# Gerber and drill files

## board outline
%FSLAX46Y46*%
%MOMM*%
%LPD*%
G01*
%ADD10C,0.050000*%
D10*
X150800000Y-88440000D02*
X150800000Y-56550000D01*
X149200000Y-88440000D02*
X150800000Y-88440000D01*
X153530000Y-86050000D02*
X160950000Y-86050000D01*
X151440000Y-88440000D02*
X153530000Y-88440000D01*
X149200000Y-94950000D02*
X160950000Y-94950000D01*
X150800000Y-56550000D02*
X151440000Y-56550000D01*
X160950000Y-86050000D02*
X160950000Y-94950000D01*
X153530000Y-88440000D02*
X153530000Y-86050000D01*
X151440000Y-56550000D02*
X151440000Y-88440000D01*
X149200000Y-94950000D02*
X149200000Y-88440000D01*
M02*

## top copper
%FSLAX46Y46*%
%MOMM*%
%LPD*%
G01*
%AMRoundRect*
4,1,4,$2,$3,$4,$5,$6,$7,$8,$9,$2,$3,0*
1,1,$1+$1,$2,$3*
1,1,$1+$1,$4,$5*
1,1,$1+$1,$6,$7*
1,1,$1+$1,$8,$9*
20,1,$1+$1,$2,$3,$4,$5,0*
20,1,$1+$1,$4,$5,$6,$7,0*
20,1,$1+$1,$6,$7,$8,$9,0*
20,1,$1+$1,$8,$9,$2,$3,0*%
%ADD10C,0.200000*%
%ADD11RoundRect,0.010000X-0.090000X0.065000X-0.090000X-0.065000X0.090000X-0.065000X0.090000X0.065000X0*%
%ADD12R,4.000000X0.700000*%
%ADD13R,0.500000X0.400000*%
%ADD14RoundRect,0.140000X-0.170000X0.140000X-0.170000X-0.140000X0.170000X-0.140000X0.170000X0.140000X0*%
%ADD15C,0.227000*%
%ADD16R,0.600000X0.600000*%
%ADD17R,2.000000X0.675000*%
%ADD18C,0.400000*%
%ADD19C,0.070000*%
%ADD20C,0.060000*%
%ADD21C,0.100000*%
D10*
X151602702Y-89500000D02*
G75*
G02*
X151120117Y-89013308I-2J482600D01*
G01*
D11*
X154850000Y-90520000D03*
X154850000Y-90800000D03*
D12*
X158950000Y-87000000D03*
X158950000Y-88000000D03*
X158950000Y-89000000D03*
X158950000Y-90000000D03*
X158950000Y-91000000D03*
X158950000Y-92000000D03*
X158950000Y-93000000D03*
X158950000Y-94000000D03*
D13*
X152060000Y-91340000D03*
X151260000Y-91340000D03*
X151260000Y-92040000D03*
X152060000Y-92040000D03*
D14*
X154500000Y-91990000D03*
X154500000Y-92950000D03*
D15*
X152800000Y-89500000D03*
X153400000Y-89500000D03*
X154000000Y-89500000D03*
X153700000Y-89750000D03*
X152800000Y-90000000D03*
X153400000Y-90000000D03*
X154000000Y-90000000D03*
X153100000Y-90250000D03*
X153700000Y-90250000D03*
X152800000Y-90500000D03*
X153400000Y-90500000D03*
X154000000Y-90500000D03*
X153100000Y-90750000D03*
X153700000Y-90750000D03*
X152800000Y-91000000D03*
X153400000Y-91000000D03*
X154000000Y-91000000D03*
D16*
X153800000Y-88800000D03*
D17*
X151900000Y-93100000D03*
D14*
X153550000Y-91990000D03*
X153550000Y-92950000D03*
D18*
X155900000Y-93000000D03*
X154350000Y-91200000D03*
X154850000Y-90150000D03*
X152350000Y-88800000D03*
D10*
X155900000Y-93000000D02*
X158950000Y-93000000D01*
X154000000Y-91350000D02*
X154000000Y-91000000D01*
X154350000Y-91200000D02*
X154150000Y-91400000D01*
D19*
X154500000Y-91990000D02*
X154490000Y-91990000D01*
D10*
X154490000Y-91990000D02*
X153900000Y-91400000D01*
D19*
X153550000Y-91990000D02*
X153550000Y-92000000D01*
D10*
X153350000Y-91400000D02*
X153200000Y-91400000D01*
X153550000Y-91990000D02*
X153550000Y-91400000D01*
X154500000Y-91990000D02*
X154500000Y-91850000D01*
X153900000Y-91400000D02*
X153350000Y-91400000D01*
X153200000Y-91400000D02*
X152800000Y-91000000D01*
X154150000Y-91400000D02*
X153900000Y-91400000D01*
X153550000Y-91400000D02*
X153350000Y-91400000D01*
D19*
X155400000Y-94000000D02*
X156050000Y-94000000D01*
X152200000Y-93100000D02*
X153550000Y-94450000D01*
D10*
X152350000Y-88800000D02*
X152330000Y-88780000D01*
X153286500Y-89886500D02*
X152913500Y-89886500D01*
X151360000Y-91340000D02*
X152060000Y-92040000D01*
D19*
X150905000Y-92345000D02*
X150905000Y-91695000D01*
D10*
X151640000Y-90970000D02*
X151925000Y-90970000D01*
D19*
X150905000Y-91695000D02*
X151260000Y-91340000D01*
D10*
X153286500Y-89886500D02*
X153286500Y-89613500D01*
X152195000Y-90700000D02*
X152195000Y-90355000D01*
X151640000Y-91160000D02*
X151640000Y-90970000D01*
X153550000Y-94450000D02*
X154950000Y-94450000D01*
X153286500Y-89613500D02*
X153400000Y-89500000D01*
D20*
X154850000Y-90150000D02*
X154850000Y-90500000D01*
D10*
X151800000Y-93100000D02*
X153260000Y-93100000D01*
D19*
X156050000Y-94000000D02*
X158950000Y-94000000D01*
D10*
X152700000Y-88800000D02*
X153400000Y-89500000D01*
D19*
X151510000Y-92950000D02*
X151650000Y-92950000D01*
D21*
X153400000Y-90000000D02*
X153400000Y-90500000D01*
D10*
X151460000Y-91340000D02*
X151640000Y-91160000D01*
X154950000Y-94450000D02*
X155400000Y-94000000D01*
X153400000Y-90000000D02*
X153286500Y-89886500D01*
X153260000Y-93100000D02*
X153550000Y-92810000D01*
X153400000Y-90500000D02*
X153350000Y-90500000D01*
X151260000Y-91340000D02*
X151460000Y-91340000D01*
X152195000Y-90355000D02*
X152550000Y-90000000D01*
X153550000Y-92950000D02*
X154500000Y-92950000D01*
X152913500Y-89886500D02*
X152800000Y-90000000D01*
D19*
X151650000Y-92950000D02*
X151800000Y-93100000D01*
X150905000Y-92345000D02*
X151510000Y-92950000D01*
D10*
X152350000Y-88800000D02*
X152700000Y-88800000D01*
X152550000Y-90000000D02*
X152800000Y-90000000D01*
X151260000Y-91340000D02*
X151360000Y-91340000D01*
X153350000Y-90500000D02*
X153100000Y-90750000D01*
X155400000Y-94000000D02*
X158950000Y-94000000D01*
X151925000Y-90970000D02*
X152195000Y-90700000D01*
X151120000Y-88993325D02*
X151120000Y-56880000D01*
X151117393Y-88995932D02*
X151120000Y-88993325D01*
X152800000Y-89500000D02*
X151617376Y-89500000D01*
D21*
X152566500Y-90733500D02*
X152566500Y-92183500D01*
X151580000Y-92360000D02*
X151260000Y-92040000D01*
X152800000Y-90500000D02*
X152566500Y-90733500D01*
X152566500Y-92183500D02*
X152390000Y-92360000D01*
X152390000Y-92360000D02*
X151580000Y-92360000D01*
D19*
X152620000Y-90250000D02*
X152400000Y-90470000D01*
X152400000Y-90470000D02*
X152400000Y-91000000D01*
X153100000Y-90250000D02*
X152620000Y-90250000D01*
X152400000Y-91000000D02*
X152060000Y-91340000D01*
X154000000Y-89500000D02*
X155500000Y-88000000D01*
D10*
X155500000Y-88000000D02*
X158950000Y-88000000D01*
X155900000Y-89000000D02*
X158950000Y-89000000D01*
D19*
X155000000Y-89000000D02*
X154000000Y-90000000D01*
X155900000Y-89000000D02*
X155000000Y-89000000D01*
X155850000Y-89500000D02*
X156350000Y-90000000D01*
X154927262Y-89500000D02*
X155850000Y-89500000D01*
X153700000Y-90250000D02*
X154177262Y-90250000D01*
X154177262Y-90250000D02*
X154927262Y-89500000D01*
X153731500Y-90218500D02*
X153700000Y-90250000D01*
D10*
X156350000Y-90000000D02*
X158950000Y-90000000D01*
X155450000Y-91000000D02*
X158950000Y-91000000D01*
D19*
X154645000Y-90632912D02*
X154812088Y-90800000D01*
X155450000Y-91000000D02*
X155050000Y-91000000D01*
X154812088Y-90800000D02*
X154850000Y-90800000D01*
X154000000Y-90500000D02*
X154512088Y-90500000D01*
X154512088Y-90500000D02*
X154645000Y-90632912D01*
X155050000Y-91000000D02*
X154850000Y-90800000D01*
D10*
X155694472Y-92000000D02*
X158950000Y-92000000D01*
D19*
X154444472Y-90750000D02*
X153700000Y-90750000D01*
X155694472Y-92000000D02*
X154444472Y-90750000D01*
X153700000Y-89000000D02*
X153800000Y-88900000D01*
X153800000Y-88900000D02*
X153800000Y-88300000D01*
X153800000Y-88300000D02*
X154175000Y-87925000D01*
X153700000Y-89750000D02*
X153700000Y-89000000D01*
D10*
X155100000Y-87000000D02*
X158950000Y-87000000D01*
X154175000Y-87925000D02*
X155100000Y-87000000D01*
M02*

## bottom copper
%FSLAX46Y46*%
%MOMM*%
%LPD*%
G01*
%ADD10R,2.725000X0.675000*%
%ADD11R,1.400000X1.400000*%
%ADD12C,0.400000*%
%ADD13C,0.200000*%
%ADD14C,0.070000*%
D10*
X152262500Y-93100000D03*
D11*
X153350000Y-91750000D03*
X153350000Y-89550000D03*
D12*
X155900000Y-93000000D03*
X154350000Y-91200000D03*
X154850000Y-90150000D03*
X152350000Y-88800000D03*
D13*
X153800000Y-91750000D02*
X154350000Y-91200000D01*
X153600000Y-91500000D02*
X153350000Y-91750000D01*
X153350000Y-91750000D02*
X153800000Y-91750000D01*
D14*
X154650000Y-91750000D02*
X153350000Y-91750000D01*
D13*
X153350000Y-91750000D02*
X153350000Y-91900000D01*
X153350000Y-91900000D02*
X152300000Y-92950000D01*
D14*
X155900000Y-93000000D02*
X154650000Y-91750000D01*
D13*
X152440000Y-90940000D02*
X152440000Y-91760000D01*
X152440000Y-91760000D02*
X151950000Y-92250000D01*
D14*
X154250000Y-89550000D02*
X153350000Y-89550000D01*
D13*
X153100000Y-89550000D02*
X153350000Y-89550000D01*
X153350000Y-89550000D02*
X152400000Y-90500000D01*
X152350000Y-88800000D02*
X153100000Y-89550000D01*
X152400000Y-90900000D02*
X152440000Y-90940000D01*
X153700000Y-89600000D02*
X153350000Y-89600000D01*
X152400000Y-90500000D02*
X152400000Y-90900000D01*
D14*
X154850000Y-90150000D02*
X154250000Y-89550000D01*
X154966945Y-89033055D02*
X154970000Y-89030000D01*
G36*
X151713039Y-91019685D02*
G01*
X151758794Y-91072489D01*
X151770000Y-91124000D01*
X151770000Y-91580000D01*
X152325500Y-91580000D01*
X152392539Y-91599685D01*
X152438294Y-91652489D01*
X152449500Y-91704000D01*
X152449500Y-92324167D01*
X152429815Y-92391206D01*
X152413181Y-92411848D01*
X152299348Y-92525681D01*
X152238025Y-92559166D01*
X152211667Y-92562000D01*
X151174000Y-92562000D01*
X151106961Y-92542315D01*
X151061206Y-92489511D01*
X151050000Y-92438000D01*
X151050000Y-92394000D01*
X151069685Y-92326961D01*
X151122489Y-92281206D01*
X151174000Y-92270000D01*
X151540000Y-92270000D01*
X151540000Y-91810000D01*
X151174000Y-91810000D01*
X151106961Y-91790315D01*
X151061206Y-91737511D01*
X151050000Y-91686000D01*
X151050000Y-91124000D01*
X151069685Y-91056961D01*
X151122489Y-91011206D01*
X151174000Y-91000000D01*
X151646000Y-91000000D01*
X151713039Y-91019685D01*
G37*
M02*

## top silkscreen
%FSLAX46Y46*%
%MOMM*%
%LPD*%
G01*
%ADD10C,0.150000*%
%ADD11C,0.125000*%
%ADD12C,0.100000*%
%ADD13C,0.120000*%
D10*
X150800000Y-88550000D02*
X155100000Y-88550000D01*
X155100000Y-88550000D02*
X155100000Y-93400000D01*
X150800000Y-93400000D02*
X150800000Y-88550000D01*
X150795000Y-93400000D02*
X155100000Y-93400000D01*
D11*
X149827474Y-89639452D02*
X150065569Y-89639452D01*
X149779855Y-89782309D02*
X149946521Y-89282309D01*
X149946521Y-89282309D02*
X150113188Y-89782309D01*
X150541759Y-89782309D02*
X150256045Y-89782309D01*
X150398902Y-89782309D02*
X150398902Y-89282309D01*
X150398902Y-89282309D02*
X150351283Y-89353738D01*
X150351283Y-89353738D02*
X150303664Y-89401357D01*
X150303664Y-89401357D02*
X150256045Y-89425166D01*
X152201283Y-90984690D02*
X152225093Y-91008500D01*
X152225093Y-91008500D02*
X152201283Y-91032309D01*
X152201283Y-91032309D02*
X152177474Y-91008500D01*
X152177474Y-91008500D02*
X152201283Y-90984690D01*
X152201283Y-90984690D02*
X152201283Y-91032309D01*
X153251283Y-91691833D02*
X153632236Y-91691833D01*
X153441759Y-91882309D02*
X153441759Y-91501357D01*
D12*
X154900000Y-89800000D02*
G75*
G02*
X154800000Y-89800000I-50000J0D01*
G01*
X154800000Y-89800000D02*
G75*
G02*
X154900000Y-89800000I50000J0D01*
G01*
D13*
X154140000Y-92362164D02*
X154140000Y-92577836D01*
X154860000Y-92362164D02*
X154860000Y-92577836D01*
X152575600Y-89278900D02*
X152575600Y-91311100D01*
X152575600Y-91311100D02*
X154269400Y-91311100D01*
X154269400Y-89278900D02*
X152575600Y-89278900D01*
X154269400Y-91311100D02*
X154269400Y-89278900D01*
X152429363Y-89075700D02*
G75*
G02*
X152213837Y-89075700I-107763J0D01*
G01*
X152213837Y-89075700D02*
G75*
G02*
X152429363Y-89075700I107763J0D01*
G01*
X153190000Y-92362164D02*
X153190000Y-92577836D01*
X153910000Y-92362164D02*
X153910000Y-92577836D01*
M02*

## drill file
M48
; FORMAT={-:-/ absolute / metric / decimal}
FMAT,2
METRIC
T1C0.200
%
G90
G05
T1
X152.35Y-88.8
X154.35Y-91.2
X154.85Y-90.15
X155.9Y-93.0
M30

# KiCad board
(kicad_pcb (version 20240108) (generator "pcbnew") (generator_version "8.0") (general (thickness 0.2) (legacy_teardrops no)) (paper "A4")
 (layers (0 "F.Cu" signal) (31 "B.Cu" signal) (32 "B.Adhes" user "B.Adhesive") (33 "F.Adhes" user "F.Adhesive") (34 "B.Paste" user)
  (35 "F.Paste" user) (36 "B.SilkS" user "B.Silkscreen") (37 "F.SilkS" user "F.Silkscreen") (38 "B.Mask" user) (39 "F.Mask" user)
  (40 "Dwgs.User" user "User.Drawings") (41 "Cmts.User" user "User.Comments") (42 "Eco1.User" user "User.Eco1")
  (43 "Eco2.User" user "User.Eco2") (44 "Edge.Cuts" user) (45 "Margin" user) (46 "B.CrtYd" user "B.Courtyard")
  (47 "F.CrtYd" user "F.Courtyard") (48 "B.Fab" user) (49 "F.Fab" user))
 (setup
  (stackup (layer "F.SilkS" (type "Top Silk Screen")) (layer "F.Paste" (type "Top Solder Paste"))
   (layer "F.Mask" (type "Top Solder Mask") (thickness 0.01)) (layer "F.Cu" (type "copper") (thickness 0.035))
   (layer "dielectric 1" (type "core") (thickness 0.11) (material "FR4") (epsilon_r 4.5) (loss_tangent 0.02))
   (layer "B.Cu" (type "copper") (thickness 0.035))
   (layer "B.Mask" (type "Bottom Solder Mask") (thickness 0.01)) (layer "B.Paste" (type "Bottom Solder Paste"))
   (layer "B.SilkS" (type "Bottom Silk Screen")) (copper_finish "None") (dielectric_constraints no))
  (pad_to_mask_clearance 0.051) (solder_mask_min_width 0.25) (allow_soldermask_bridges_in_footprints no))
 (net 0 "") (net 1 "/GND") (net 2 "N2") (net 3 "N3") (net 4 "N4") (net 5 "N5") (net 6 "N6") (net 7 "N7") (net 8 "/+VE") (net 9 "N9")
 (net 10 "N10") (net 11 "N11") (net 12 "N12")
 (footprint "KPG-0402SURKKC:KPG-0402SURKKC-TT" (layer "F.Cu") (at 154.85 90.66 -90)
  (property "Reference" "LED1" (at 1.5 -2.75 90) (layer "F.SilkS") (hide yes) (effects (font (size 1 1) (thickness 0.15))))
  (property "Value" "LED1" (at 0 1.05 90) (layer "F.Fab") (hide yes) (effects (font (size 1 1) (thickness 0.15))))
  (fp_circle (center -0.86 0) (end -0.81 0) (stroke (width 0.1) (type solid)) (fill none) (layer "F.SilkS"))
  (pad "" smd roundrect (at -0.14 0 270) (size 0.15 0.2) (layers "F.Mask") (roundrect_rratio 0.06666666667))
  (pad "" smd roundrect (at -0.1225 0 270) (size 0.1 0.17) (layers "F.Paste") (roundrect_rratio 0.25))
  (pad "" smd roundrect (at 0.1225 0 270) (size 0.1 0.17) (layers "F.Paste") (roundrect_rratio 0.25))
  (pad "" smd roundrect (at 0.14 0 270) (size 0.15 0.2) (layers "F.Mask") (roundrect_rratio 0.06666666667))
  (pad "1" smd roundrect (at -0.14 0 270) (size 0.15 0.2) (layers "F.Cu" "F.Mask") (roundrect_rratio 0.06666666667) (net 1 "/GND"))
  (pad "2" smd roundrect (at 0.14 0 270) (size 0.15 0.2) (layers "F.Cu" "F.Mask") (roundrect_rratio 0.06666666667) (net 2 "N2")))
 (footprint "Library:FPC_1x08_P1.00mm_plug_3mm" (layer "F.Cu") (at 156.95 90.5)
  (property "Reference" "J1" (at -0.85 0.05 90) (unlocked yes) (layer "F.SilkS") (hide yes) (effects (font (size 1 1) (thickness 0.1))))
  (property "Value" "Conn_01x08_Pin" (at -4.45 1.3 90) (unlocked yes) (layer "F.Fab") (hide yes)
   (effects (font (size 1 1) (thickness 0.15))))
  (pad "1" connect rect (at 2 -3.5) (size 4 0.7) (layers "F.Cu" "F.Mask") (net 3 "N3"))
  (pad "2" connect rect (at 2 -2.5) (size 4 0.7) (layers "F.Cu" "F.Mask") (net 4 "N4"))
  (pad "3" connect rect (at 2 -1.5) (size 4 0.7) (layers "F.Cu" "F.Mask") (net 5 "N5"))
  (pad "4" connect rect (at 2 -0.5) (size 4 0.7) (layers "F.Cu" "F.Mask") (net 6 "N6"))
  (pad "5" connect rect (at 2 0.5) (size 4 0.7) (layers "F.Cu" "F.Mask") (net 2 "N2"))
  (pad "6" connect rect (at 2 1.5) (size 4 0.7) (layers "F.Cu" "F.Mask") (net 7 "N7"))
  (pad "7" connect rect (at 2 2.5) (size 4 0.7) (layers "F.Cu" "F.Mask") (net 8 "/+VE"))
  (pad "8" connect rect (at 2 3.5) (size 4 0.7) (layers "F.Cu" "F.Mask") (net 1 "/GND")))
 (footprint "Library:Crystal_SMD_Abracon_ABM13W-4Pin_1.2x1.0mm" (layer "F.Cu") (at 151.66 91.69 180)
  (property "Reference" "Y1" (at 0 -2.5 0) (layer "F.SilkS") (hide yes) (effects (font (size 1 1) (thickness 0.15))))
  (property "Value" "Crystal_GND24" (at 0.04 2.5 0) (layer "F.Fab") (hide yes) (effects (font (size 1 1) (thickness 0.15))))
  (pad "1" smd rect (at -0.4 0.35 180) (size 0.5 0.4) (layers "F.Cu" "F.Paste" "F.Mask") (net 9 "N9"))
  (pad "2" smd rect (at 0.4 0.35 180) (size 0.5 0.4) (layers "F.Cu" "F.Paste" "F.Mask") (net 1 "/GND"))
  (pad "3" smd rect (at 0.4 -0.35 180) (size 0.5 0.4) (layers "F.Cu" "F.Paste" "F.Mask") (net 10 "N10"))
  (pad "4" smd rect (at -0.4 -0.35 180) (size 0.5 0.4) (layers "F.Cu" "F.Paste" "F.Mask") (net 1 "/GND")))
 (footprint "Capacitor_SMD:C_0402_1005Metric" (layer "F.Cu") (at 154.5 92.47 -90)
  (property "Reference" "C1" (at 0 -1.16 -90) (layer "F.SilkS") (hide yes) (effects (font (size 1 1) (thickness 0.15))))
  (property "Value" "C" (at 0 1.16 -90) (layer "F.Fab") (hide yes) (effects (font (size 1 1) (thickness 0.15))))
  (fp_line (start -0.107836 0.36) (end 0.107836 0.36) (stroke (width 0.12) (type solid)) (layer "F.SilkS"))
  (fp_line (start -0.107836 -0.36) (end 0.107836 -0.36) (stroke (width 0.12) (type solid)) (layer "F.SilkS"))
  (pad "1" smd roundrect (at -0.48 0 270) (size 0.56 0.62) (layers "F.Cu" "F.Paste" "F.Mask") (roundrect_rratio 0.25) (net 8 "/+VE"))
  (pad "2" smd roundrect (at 0.48 0 270) (size 0.56 0.62) (layers "F.Cu" "F.Paste" "F.Mask") (roundrect_rratio 0.25) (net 1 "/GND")))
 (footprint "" (layer "F.Cu") (at 152.15 93.3625)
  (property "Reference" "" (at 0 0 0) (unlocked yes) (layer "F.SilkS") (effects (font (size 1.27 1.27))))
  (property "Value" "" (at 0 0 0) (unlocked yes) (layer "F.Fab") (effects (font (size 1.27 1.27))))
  (pad "2" smd rect (at 0.1125 -0.2625 270) (size 0.675 2.725) (layers "B.Cu" "B.Paste" "B.Mask") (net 8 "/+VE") (solder_mask_margin 0.102)))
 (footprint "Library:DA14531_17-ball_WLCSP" (layer "F.Cu") (at 153.422 90.295)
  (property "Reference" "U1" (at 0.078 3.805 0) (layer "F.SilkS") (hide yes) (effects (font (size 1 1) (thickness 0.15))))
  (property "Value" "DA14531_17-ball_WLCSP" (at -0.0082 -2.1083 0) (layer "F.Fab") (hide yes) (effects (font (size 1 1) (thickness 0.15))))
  (fp_line (start -0.8464 -1.0161) (end -0.8464 1.0161) (stroke (width 0.12) (type solid)) (layer "F.SilkS"))
  (fp_line (start -0.8464 1.0161) (end 0.8474 1.0161) (stroke (width 0.12) (type solid)) (layer "F.SilkS"))
  (fp_line (start 0.8474 -1.0161) (end -0.8464 -1.0161) (stroke (width 0.12) (type solid)) (layer "F.SilkS"))
  (fp_line (start 0.8474 1.0161) (end 0.8474 -1.0161) (stroke (width 0.12) (type solid)) (layer "F.SilkS"))
  (fp_circle (center -1.1004 -1.2193) (end -1.0242 -1.1431) (stroke (width 0.12) (type solid)) (fill none) (layer "F.SilkS"))
  (pad "A1" smd circle (at -0.622 -0.795) (size 0.227 0.227) (layers "F.Cu" "F.Paste" "F.Mask") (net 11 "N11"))
  (pad "A3" smd circle (at -0.022 -0.795) (size 0.227 0.227) (layers "F.Cu" "F.Paste" "F.Mask") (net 1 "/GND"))
  (pad "A5" smd circle (at 0.578 -0.795) (size 0.227 0.227) (layers "F.Cu" "F.Paste" "F.Mask") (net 4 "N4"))
  (pad "B4" smd circle (at 0.278 -0.545) (size 0.227 0.227) (layers "F.Cu" "F.Paste" "F.Mask") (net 3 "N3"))
  (pad "C1" smd circle (at -0.622 -0.295) (size 0.227 0.227) (layers "F.Cu" "F.Paste" "F.Mask") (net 1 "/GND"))
  (pad "C3" smd circle (at -0.022 -0.295) (size 0.227 0.227) (layers "F.Cu" "F.Paste" "F.Mask") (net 1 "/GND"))
  (pad "C5" smd circle (at 0.578 -0.295) (size 0.227 0.227) (layers "F.Cu" "F.Paste" "F.Mask") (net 5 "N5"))
  (pad "D2" smd circle (at -0.322 -0.045) (size 0.227 0.227) (layers "F.Cu" "F.Paste" "F.Mask") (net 9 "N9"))
  (pad "D4" smd circle (at 0.278 -0.045) (size 0.227 0.227) (layers "F.Cu" "F.Paste" "F.Mask") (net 6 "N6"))
  (pad "E1" smd circle (at -0.622 0.205) (size 0.227 0.227) (layers "F.Cu" "F.Paste" "F.Mask") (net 10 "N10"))
  (pad "E3" smd circle (at -0.022 0.205) (size 0.227 0.227) (layers "F.Cu" "F.Paste" "F.Mask") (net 1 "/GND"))
  (pad "E5" smd circle (at 0.578 0.205) (size 0.227 0.227) (layers "F.Cu" "F.Paste" "F.Mask") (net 2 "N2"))
  (pad "F2" smd circle (at -0.322 0.455) (size 0.227 0.227) (layers "F.Cu" "F.Paste" "F.Mask") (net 1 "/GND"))
  (pad "F4" smd circle (at 0.278 0.455) (size 0.227 0.227) (layers "F.Cu" "F.Paste" "F.Mask") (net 7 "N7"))
  (pad "G1" smd circle (at -0.622 0.705) (size 0.227 0.227) (layers "F.Cu" "F.Paste" "F.Mask") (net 8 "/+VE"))
  (pad "G3" smd circle (at -0.022 0.705) (size 0.227 0.227) (layers "F.Cu" "F.Paste" "F.Mask") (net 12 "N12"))
  (pad "G5" smd circle (at 0.578 0.705) (size 0.227 0.227) (layers "F.Cu" "F.Paste" "F.Mask") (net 8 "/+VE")))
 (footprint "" (layer "F.Cu") (at 153.4 89.1)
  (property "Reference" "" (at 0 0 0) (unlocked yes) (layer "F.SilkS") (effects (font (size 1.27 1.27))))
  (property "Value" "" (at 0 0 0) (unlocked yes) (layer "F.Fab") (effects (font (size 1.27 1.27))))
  (pad "2" smd rect (at 0.4 -0.3 270) (size 0.6 0.6) (layers "F.Cu" "F.Paste" "F.Mask") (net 3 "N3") (solder_mask_margin 0.102)))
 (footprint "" (layer "F.Cu") (at 151.8 93.2)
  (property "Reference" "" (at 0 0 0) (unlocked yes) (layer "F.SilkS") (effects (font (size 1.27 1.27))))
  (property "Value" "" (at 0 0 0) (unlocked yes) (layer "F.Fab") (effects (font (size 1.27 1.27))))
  (pad "2" smd rect (at 0.1 -0.1 270) (size 0.675 2) (layers "F.Cu" "F.Paste" "F.Mask") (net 1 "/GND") (solder_mask_margin 0.102)))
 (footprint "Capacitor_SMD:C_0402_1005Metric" (layer "F.Cu") (at 153.55 92.47 -90)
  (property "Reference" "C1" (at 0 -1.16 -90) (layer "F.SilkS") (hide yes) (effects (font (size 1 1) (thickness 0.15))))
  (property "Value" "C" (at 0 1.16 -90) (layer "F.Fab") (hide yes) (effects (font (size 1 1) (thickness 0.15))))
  (fp_line (start -0.107836 0.36) (end 0.107836 0.36) (stroke (width 0.12) (type solid)) (layer "F.SilkS"))
  (fp_line (start -0.107836 -0.36) (end 0.107836 -0.36) (stroke (width 0.12) (type solid)) (layer "F.SilkS"))
  (pad "1" smd roundrect (at -0.48 0 270) (size 0.56 0.62) (layers "F.Cu" "F.Paste" "F.Mask") (roundrect_rratio 0.25) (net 8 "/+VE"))
  (pad "2" smd roundrect (at 0.48 0 270) (size 0.56 0.62) (layers "F.Cu" "F.Paste" "F.Mask") (roundrect_rratio 0.25) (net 1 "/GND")))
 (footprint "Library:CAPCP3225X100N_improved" (layer "B.Cu") (at 153.35 90.65 90)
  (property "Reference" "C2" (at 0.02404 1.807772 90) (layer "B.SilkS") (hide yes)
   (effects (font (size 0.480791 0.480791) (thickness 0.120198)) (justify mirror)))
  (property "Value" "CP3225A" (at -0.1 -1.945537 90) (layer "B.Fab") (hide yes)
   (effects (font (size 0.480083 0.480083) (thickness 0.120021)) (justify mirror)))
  (pad "1" smd rect (at -1.1 0 270) (size 1.4 1.4) (layers "B.Cu" "B.Paste" "B.Mask") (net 8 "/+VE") (solder_mask_margin 0.102))
  (pad "2" smd rect (at 1.1 0 270) (size 1.4 1.4) (layers "B.Cu" "B.Paste" "B.Mask") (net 1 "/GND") (solder_mask_margin 0.102)))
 (gr_arc (start 151.602702 89.5) (mid 151.26 89.357201) (end 151.120095 89.013308) (stroke (width 0.2) (type default)) (layer "F.Cu")
  (net 11))
 (gr_line (start 150.8 88.55) (end 155.1 88.55) (stroke (width 0.15) (type default)) (layer "F.SilkS"))
 (gr_line (start 155.1 88.55) (end 155.1 93.4) (stroke (width 0.15) (type default)) (layer "F.SilkS"))
 (gr_line (start 150.8 93.4) (end 150.8 88.55) (stroke (width 0.15) (type default)) (layer "F.SilkS"))
 (gr_line (start 150.795 93.4) (end 155.1 93.4) (stroke (width 0.15) (type default)) (layer "F.SilkS"))
 (gr_line (start 150.8 88.44) (end 150.8 56.55) (stroke (width 0.05) (type default)) (layer "Edge.Cuts"))
 (gr_line (start 149.2 88.44) (end 150.8 88.44) (stroke (width 0.05) (type default)) (layer "Edge.Cuts"))
 (gr_line (start 153.53 86.05) (end 160.95 86.05) (stroke (width 0.05) (type default)) (layer "Edge.Cuts"))
 (gr_line (start 151.44 88.44) (end 153.53 88.44) (stroke (width 0.05) (type default)) (layer "Edge.Cuts"))
 (gr_line (start 149.2 94.95) (end 160.95 94.95) (stroke (width 0.05) (type default)) (layer "Edge.Cuts"))
 (gr_line (start 150.8 56.55) (end 151.44 56.55) (stroke (width 0.05) (type default)) (layer "Edge.Cuts"))
 (gr_line (start 160.95 86.05) (end 160.95 94.95) (stroke (width 0.05) (type default)) (layer "Edge.Cuts"))
 (gr_line (start 153.53 88.44) (end 153.53 86.05) (stroke (width 0.05) (type default)) (layer "Edge.Cuts"))
 (gr_line (start 151.44 56.55) (end 151.44 88.44) (stroke (width 0.05) (type default)) (layer "Edge.Cuts"))
 (gr_line (start 149.2 94.95) (end 149.2 88.44) (stroke (width 0.05) (type default)) (layer "Edge.Cuts"))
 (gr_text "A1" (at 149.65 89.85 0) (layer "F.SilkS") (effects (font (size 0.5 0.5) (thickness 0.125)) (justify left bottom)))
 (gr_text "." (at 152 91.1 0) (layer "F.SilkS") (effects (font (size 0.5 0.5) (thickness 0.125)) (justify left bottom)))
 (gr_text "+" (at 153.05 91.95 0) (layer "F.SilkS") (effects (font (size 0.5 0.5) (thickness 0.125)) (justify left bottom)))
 (segment (start 155.9 93) (end 158.95 93) (width 0.2) (layer "F.Cu") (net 8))
 (segment (start 154 91.35) (end 154 91) (width 0.2) (layer "F.Cu") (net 8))
 (segment (start 154.35 91.2) (end 154.15 91.4) (width 0.2) (layer "F.Cu") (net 8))
 (segment (start 154.5 91.99) (end 154.49 91.99) (width 0.07) (layer "F.Cu") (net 8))
 (segment (start 154.49 91.99) (end 153.9 91.4) (width 0.2) (layer "F.Cu") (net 8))
 (segment (start 153.55 91.99) (end 153.55 92) (width 0.07) (layer "F.Cu") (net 8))
 (segment (start 153.35 91.4) (end 153.2 91.4) (width 0.2) (layer "F.Cu") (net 8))
 (segment (start 153.55 91.99) (end 153.55 91.4) (width 0.2) (layer "F.Cu") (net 8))
 (segment (start 154.5 91.99) (end 154.5 91.85) (width 0.2) (layer "F.Cu") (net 8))
 (segment (start 153.9 91.4) (end 153.35 91.4) (width 0.2) (layer "F.Cu") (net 8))
 (segment (start 153.2 91.4) (end 152.8 91) (width 0.2) (layer "F.Cu") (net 8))
 (segment (start 154.15 91.4) (end 153.9 91.4) (width 0.2) (layer "F.Cu") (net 8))
 (segment (start 153.55 91.4) (end 153.35 91.4) (width 0.2) (layer "F.Cu") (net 8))
 (via (at 155.9 93) (size 0.4) (drill 0.2) (layers "F.Cu" "B.Cu") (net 8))
 (via (at 154.35 91.2) (size 0.4) (drill 0.2) (layers "F.Cu" "B.Cu") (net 8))
 (segment (start 153.8 91.75) (end 154.35 91.2) (width 0.2) (layer "B.Cu") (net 8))
 (segment (start 153.6 91.5) (end 153.35 91.75) (width 0.2) (layer "B.Cu") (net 8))
 (segment (start 153.35 91.75) (end 153.8 91.75) (width 0.2) (layer "B.Cu") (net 8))
 (segment (start 154.65 91.75) (end 153.35 91.75) (width 0.07) (layer "B.Cu") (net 8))
 (segment (start 153.35 91.75) (end 153.35 91.9) (width 0.2) (layer "B.Cu") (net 8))
 (segment (start 153.35 91.9) (end 152.3 92.95) (width 0.2) (layer "B.Cu") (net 8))
 (segment (start 155.9 93) (end 154.65 91.75) (width 0.07) (layer "B.Cu") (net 8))
 (segment (start 155.4 94) (end 156.05 94) (width 0.07) (layer "F.Cu") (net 1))
 (segment (start 152.2 93.1) (end 153.55 94.45) (width 0.07) (layer "F.Cu") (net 1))
 (segment (start 152.35 88.8) (end 152.33 88.78) (width 0.2) (layer "F.Cu") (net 1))
 (segment (start 153.2865 89.8865) (end 152.9135 89.8865) (width 0.2) (layer "F.Cu") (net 1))
 (segment (start 151.36 91.34) (end 152.06 92.04) (width 0.2) (layer "F.Cu") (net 1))
 (segment (start 150.905 92.345) (end 150.905 91.695) (width 0.07) (layer "F.Cu") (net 1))
 (segment (start 151.64 90.97) (end 151.925 90.97) (width 0.2) (layer "F.Cu") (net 1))
 (segment (start 150.905 91.695) (end 151.26 91.34) (width 0.07) (layer "F.Cu") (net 1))
 (segment (start 153.2865 89.8865) (end 153.2865 89.6135) (width 0.2) (layer "F.Cu") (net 1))
 (segment (start 152.195 90.7) (end 152.195 90.355) (width 0.2) (layer "F.Cu") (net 1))
 (segment (start 151.64 91.16) (end 151.64 90.97) (width 0.2) (layer "F.Cu") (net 1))
 (segment (start 153.55 94.45) (end 154.95 94.45) (width 0.2) (layer "F.Cu") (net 1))
 (segment (start 153.2865 89.6135) (end 153.4 89.5) (width 0.2) (layer "F.Cu") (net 1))
 (segment (start 154.85 90.15) (end 154.85 90.5) (width 0.06) (layer "F.Cu") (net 1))
 (segment (start 151.8 93.1) (end 153.26 93.1) (width 0.2) (layer "F.Cu") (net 1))
 (segment (start 156.05 94) (end 158.95 94) (width 0.07) (layer "F.Cu") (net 1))
 (segment (start 152.7 88.8) (end 153.4 89.5) (width 0.2) (layer "F.Cu") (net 1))
 (segment (start 151.51 92.95) (end 151.65 92.95) (width 0.07) (layer "F.Cu") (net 1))
 (segment (start 153.4 90) (end 153.4 90.5) (width 0.1) (layer "F.Cu") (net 1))
 (segment (start 151.46 91.34) (end 151.64 91.16) (width 0.2) (layer "F.Cu") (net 1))
 (segment (start 154.95 94.45) (end 155.4 94) (width 0.2) (layer "F.Cu") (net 1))
 (segment (start 153.4 90) (end 153.2865 89.8865) (width 0.2) (layer "F.Cu") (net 1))
 (segment (start 153.26 93.1) (end 153.55 92.81) (width 0.2) (layer "F.Cu") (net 1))
 (segment (start 153.4 90.5) (end 153.35 90.5) (width 0.2) (layer "F.Cu") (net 1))
 (segment (start 151.26 91.34) (end 151.46 91.34) (width 0.2) (layer "F.Cu") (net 1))
 (segment (start 152.195 90.355) (end 152.55 90) (width 0.2) (layer "F.Cu") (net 1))
 (segment (start 153.55 92.95) (end 154.5 92.95) (width 0.2) (layer "F.Cu") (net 1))
 (segment (start 152.9135 89.8865) (end 152.8 90) (width 0.2) (layer "F.Cu") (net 1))
 (segment (start 151.65 92.95) (end 151.8 93.1) (width 0.07) (layer "F.Cu") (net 1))
 (segment (start 150.905 92.345) (end 151.51 92.95) (width 0.07) (layer "F.Cu") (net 1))
 (segment (start 152.35 88.8) (end 152.7 88.8) (width 0.2) (layer "F.Cu") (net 1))
 (segment (start 152.55 90) (end 152.8 90) (width 0.2) (layer "F.Cu") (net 1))
 (segment (start 151.26 91.34) (end 151.36 91.34) (width 0.2) (layer "F.Cu") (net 1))
 (segment (start 153.35 90.5) (end 153.1 90.75) (width 0.2) (layer "F.Cu") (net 1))
 (segment (start 155.4 94) (end 158.95 94) (width 0.2) (layer "F.Cu") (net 1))
 (segment (start 151.925 90.97) (end 152.195 90.7) (width 0.2) (layer "F.Cu") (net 1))
 (via (at 154.85 90.15) (size 0.4) (drill 0.2) (layers "F.Cu" "B.Cu") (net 1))
 (via (at 152.35 88.8) (size 0.4) (drill 0.2) (layers "F.Cu" "B.Cu") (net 1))
 (segment (start 152.44 90.94) (end 152.44 91.76) (width 0.2) (layer "B.Cu") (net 1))
 (segment (start 152.44 91.76) (end 151.95 92.25) (width 0.2) (layer "B.Cu") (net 1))
 (segment (start 154.25 89.55) (end 153.35 89.55) (width 0.07) (layer "B.Cu") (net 1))
 (segment (start 153.1 89.55) (end 153.35 89.55) (width 0.2) (layer "B.Cu") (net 1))
 (segment (start 153.35 89.55) (end 152.4 90.5) (width 0.2) (layer "B.Cu") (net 1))
 (segment (start 152.35 88.8) (end 153.1 89.55) (width 0.2) (layer "B.Cu") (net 1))
 (segment (start 152.4 90.9) (end 152.44 90.94) (width 0.2) (layer "B.Cu") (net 1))
 (segment (start 153.7 89.6) (end 153.35 89.6) (width 0.2) (layer "B.Cu") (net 1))
 (segment (start 152.4 90.5) (end 152.4 90.9) (width 0.2) (layer "B.Cu") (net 1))
 (segment (start 154.85 90.15) (end 154.25 89.55) (width 0.07) (layer "B.Cu") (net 1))
 (segment (start 151.12 88.993325) (end 151.12 56.88) (width 0.2) (layer "F.Cu") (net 11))
 (segment (start 151.117393 88.995932) (end 151.12 88.993325) (width 0.2) (layer "F.Cu") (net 11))
 (segment (start 152.8 89.5) (end 151.617376 89.5) (width 0.2) (layer "F.Cu") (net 11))
 (segment (start 152.5665 90.7335) (end 152.5665 92.1835) (width 0.1) (layer "F.Cu") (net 10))
 (segment (start 151.58 92.36) (end 151.26 92.04) (width 0.1) (layer "F.Cu") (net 10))
 (segment (start 152.8 90.5) (end 152.5665 90.7335) (width 0.1) (layer "F.Cu") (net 10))
 (segment (start 152.5665 92.1835) (end 152.39 92.36) (width 0.1) (layer "F.Cu") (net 10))
 (segment (start 152.39 92.36) (end 151.58 92.36) (width 0.1) (layer "F.Cu") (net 10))
 (segment (start 152.62 90.25) (end 152.4 90.47) (width 0.07) (layer "F.Cu") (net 9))
 (segment (start 152.4 90.47) (end 152.4 91) (width 0.07) (layer "F.Cu") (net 9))
 (segment (start 153.1 90.25) (end 152.62 90.25) (width 0.07) (layer "F.Cu") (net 9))
 (segment (start 152.4 91) (end 152.06 91.34) (width 0.07) (layer "F.Cu") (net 9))
 (segment (start 154 89.5) (end 155.5 88) (width 0.07) (layer "F.Cu") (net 4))
 (segment (start 155.5 88) (end 158.95 88) (width 0.2) (layer "F.Cu") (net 4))
 (segment (start 155.9 89) (end 158.95 89) (width 0.2) (layer "F.Cu") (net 5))
 (segment (start 155 89) (end 154 90) (width 0.07) (layer "F.Cu") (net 5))
 (segment (start 155.9 89) (end 155 89) (width 0.07) (layer "F.Cu") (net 5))
 (segment (start 154.966945 89.033055) (end 154.97 89.03) (width 0.07) (layer "B.Cu") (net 5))
 (segment (start 155.85 89.5) (end 156.35 90) (width 0.07) (layer "F.Cu") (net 6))
 (segment (start 154.927262 89.5) (end 155.85 89.5) (width 0.07) (layer "F.Cu") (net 6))
 (segment (start 153.7 90.25) (end 154.177262 90.25) (width 0.07) (layer "F.Cu") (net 6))
 (segment (start 154.177262 90.25) (end 154.927262 89.5) (width 0.07) (layer "F.Cu") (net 6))
 (segment (start 153.7315 90.2185) (end 153.7 90.25) (width 0.07) (layer "F.Cu") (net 6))
 (segment (start 156.35 90) (end 158.95 90) (width 0.2) (layer "F.Cu") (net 6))
 (segment (start 155.45 91) (end 158.95 91) (width 0.2) (layer "F.Cu") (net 2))
 (segment (start 154.645 90.632912) (end 154.812088 90.8) (width 0.07) (layer "F.Cu") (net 2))
 (segment (start 155.45 91) (end 155.05 91) (width 0.07) (layer "F.Cu") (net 2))
 (segment (start 154.812088 90.8) (end 154.85 90.8) (width 0.07) (layer "F.Cu") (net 2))
 (segment (start 154 90.5) (end 154.512088 90.5) (width 0.07) (layer "F.Cu") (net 2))
 (segment (start 154.512088 90.5) (end 154.645 90.632912) (width 0.07) (layer "F.Cu") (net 2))
 (segment (start 155.05 91) (end 154.85 90.8) (width 0.07) (layer "F.Cu") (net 2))
 (segment (start 155.694472 92) (end 158.95 92) (width 0.2) (layer "F.Cu") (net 7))
 (segment (start 154.444472 90.75) (end 153.7 90.75) (width 0.07) (layer "F.Cu") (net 7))
 (segment (start 155.694472 92) (end 154.444472 90.75) (width 0.07) (layer "F.Cu") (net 7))
 (segment (start 153.7 89) (end 153.8 88.9) (width 0.07) (layer "F.Cu") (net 3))
 (segment (start 153.8 88.9) (end 153.8 88.3) (width 0.07) (layer "F.Cu") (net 3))
 (segment (start 153.8 88.3) (end 154.175 87.925) (width 0.07) (layer "F.Cu") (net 3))
 (segment (start 153.7 89.75) (end 153.7 89) (width 0.07) (layer "F.Cu") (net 3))
 (segment (start 155.1 87) (end 158.95 87) (width 0.2) (layer "F.Cu") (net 3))
 (segment (start 154.175 87.925) (end 155.1 87) (width 0.2) (layer "F.Cu") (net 3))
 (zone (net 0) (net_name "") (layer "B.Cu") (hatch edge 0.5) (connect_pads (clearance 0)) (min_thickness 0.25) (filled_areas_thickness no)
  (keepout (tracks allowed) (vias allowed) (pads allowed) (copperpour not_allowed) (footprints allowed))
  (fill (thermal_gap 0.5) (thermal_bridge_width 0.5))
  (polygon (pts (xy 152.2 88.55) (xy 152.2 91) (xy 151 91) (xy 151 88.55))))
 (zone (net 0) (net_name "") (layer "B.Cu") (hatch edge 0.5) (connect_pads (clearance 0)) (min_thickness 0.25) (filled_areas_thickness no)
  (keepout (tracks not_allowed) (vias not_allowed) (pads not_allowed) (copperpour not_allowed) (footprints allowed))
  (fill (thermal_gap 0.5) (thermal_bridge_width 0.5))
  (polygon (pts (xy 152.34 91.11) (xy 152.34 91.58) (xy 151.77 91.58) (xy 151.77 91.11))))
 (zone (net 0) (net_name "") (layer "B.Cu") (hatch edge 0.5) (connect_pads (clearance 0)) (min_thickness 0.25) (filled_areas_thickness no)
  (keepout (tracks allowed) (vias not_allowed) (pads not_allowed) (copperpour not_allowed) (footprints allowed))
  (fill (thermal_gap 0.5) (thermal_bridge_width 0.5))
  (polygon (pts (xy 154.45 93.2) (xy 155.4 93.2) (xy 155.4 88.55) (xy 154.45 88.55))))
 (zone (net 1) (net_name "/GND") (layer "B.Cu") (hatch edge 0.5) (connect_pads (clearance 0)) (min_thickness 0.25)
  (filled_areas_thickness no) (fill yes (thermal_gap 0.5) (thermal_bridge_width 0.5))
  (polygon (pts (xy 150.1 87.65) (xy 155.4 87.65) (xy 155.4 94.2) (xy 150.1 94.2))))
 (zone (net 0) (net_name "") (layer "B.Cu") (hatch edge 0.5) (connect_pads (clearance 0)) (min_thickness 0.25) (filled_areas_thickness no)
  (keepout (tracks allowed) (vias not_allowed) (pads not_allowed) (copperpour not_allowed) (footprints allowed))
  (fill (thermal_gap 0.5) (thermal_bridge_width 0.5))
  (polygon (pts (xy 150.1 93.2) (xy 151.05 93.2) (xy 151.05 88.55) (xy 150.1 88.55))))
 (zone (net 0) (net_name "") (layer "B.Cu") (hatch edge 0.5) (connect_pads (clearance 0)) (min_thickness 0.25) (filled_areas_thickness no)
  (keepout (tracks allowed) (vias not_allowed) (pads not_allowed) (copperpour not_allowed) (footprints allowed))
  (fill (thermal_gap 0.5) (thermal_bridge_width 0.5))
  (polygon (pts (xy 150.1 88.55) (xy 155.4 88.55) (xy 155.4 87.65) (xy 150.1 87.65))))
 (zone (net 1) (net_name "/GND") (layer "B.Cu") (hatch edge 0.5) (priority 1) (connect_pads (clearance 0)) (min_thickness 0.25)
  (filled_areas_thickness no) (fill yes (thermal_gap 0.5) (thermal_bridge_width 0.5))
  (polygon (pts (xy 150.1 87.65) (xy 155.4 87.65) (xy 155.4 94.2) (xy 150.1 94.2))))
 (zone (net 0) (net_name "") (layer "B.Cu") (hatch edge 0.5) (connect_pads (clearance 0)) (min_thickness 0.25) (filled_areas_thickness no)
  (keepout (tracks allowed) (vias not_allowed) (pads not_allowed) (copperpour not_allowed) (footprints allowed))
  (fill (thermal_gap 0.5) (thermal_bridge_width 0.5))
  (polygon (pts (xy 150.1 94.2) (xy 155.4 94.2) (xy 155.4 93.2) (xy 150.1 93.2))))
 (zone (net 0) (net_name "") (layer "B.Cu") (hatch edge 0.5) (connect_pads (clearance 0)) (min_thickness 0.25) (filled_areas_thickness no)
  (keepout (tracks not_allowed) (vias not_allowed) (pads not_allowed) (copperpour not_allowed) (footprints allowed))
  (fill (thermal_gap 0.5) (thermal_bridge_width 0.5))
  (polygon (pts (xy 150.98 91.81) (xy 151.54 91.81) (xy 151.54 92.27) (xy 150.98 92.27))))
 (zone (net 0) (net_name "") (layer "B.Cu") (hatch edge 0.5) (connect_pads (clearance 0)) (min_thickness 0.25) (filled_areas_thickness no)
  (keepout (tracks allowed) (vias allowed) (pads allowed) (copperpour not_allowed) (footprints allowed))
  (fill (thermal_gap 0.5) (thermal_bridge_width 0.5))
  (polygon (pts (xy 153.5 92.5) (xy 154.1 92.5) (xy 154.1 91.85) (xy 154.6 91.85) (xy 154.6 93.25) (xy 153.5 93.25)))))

